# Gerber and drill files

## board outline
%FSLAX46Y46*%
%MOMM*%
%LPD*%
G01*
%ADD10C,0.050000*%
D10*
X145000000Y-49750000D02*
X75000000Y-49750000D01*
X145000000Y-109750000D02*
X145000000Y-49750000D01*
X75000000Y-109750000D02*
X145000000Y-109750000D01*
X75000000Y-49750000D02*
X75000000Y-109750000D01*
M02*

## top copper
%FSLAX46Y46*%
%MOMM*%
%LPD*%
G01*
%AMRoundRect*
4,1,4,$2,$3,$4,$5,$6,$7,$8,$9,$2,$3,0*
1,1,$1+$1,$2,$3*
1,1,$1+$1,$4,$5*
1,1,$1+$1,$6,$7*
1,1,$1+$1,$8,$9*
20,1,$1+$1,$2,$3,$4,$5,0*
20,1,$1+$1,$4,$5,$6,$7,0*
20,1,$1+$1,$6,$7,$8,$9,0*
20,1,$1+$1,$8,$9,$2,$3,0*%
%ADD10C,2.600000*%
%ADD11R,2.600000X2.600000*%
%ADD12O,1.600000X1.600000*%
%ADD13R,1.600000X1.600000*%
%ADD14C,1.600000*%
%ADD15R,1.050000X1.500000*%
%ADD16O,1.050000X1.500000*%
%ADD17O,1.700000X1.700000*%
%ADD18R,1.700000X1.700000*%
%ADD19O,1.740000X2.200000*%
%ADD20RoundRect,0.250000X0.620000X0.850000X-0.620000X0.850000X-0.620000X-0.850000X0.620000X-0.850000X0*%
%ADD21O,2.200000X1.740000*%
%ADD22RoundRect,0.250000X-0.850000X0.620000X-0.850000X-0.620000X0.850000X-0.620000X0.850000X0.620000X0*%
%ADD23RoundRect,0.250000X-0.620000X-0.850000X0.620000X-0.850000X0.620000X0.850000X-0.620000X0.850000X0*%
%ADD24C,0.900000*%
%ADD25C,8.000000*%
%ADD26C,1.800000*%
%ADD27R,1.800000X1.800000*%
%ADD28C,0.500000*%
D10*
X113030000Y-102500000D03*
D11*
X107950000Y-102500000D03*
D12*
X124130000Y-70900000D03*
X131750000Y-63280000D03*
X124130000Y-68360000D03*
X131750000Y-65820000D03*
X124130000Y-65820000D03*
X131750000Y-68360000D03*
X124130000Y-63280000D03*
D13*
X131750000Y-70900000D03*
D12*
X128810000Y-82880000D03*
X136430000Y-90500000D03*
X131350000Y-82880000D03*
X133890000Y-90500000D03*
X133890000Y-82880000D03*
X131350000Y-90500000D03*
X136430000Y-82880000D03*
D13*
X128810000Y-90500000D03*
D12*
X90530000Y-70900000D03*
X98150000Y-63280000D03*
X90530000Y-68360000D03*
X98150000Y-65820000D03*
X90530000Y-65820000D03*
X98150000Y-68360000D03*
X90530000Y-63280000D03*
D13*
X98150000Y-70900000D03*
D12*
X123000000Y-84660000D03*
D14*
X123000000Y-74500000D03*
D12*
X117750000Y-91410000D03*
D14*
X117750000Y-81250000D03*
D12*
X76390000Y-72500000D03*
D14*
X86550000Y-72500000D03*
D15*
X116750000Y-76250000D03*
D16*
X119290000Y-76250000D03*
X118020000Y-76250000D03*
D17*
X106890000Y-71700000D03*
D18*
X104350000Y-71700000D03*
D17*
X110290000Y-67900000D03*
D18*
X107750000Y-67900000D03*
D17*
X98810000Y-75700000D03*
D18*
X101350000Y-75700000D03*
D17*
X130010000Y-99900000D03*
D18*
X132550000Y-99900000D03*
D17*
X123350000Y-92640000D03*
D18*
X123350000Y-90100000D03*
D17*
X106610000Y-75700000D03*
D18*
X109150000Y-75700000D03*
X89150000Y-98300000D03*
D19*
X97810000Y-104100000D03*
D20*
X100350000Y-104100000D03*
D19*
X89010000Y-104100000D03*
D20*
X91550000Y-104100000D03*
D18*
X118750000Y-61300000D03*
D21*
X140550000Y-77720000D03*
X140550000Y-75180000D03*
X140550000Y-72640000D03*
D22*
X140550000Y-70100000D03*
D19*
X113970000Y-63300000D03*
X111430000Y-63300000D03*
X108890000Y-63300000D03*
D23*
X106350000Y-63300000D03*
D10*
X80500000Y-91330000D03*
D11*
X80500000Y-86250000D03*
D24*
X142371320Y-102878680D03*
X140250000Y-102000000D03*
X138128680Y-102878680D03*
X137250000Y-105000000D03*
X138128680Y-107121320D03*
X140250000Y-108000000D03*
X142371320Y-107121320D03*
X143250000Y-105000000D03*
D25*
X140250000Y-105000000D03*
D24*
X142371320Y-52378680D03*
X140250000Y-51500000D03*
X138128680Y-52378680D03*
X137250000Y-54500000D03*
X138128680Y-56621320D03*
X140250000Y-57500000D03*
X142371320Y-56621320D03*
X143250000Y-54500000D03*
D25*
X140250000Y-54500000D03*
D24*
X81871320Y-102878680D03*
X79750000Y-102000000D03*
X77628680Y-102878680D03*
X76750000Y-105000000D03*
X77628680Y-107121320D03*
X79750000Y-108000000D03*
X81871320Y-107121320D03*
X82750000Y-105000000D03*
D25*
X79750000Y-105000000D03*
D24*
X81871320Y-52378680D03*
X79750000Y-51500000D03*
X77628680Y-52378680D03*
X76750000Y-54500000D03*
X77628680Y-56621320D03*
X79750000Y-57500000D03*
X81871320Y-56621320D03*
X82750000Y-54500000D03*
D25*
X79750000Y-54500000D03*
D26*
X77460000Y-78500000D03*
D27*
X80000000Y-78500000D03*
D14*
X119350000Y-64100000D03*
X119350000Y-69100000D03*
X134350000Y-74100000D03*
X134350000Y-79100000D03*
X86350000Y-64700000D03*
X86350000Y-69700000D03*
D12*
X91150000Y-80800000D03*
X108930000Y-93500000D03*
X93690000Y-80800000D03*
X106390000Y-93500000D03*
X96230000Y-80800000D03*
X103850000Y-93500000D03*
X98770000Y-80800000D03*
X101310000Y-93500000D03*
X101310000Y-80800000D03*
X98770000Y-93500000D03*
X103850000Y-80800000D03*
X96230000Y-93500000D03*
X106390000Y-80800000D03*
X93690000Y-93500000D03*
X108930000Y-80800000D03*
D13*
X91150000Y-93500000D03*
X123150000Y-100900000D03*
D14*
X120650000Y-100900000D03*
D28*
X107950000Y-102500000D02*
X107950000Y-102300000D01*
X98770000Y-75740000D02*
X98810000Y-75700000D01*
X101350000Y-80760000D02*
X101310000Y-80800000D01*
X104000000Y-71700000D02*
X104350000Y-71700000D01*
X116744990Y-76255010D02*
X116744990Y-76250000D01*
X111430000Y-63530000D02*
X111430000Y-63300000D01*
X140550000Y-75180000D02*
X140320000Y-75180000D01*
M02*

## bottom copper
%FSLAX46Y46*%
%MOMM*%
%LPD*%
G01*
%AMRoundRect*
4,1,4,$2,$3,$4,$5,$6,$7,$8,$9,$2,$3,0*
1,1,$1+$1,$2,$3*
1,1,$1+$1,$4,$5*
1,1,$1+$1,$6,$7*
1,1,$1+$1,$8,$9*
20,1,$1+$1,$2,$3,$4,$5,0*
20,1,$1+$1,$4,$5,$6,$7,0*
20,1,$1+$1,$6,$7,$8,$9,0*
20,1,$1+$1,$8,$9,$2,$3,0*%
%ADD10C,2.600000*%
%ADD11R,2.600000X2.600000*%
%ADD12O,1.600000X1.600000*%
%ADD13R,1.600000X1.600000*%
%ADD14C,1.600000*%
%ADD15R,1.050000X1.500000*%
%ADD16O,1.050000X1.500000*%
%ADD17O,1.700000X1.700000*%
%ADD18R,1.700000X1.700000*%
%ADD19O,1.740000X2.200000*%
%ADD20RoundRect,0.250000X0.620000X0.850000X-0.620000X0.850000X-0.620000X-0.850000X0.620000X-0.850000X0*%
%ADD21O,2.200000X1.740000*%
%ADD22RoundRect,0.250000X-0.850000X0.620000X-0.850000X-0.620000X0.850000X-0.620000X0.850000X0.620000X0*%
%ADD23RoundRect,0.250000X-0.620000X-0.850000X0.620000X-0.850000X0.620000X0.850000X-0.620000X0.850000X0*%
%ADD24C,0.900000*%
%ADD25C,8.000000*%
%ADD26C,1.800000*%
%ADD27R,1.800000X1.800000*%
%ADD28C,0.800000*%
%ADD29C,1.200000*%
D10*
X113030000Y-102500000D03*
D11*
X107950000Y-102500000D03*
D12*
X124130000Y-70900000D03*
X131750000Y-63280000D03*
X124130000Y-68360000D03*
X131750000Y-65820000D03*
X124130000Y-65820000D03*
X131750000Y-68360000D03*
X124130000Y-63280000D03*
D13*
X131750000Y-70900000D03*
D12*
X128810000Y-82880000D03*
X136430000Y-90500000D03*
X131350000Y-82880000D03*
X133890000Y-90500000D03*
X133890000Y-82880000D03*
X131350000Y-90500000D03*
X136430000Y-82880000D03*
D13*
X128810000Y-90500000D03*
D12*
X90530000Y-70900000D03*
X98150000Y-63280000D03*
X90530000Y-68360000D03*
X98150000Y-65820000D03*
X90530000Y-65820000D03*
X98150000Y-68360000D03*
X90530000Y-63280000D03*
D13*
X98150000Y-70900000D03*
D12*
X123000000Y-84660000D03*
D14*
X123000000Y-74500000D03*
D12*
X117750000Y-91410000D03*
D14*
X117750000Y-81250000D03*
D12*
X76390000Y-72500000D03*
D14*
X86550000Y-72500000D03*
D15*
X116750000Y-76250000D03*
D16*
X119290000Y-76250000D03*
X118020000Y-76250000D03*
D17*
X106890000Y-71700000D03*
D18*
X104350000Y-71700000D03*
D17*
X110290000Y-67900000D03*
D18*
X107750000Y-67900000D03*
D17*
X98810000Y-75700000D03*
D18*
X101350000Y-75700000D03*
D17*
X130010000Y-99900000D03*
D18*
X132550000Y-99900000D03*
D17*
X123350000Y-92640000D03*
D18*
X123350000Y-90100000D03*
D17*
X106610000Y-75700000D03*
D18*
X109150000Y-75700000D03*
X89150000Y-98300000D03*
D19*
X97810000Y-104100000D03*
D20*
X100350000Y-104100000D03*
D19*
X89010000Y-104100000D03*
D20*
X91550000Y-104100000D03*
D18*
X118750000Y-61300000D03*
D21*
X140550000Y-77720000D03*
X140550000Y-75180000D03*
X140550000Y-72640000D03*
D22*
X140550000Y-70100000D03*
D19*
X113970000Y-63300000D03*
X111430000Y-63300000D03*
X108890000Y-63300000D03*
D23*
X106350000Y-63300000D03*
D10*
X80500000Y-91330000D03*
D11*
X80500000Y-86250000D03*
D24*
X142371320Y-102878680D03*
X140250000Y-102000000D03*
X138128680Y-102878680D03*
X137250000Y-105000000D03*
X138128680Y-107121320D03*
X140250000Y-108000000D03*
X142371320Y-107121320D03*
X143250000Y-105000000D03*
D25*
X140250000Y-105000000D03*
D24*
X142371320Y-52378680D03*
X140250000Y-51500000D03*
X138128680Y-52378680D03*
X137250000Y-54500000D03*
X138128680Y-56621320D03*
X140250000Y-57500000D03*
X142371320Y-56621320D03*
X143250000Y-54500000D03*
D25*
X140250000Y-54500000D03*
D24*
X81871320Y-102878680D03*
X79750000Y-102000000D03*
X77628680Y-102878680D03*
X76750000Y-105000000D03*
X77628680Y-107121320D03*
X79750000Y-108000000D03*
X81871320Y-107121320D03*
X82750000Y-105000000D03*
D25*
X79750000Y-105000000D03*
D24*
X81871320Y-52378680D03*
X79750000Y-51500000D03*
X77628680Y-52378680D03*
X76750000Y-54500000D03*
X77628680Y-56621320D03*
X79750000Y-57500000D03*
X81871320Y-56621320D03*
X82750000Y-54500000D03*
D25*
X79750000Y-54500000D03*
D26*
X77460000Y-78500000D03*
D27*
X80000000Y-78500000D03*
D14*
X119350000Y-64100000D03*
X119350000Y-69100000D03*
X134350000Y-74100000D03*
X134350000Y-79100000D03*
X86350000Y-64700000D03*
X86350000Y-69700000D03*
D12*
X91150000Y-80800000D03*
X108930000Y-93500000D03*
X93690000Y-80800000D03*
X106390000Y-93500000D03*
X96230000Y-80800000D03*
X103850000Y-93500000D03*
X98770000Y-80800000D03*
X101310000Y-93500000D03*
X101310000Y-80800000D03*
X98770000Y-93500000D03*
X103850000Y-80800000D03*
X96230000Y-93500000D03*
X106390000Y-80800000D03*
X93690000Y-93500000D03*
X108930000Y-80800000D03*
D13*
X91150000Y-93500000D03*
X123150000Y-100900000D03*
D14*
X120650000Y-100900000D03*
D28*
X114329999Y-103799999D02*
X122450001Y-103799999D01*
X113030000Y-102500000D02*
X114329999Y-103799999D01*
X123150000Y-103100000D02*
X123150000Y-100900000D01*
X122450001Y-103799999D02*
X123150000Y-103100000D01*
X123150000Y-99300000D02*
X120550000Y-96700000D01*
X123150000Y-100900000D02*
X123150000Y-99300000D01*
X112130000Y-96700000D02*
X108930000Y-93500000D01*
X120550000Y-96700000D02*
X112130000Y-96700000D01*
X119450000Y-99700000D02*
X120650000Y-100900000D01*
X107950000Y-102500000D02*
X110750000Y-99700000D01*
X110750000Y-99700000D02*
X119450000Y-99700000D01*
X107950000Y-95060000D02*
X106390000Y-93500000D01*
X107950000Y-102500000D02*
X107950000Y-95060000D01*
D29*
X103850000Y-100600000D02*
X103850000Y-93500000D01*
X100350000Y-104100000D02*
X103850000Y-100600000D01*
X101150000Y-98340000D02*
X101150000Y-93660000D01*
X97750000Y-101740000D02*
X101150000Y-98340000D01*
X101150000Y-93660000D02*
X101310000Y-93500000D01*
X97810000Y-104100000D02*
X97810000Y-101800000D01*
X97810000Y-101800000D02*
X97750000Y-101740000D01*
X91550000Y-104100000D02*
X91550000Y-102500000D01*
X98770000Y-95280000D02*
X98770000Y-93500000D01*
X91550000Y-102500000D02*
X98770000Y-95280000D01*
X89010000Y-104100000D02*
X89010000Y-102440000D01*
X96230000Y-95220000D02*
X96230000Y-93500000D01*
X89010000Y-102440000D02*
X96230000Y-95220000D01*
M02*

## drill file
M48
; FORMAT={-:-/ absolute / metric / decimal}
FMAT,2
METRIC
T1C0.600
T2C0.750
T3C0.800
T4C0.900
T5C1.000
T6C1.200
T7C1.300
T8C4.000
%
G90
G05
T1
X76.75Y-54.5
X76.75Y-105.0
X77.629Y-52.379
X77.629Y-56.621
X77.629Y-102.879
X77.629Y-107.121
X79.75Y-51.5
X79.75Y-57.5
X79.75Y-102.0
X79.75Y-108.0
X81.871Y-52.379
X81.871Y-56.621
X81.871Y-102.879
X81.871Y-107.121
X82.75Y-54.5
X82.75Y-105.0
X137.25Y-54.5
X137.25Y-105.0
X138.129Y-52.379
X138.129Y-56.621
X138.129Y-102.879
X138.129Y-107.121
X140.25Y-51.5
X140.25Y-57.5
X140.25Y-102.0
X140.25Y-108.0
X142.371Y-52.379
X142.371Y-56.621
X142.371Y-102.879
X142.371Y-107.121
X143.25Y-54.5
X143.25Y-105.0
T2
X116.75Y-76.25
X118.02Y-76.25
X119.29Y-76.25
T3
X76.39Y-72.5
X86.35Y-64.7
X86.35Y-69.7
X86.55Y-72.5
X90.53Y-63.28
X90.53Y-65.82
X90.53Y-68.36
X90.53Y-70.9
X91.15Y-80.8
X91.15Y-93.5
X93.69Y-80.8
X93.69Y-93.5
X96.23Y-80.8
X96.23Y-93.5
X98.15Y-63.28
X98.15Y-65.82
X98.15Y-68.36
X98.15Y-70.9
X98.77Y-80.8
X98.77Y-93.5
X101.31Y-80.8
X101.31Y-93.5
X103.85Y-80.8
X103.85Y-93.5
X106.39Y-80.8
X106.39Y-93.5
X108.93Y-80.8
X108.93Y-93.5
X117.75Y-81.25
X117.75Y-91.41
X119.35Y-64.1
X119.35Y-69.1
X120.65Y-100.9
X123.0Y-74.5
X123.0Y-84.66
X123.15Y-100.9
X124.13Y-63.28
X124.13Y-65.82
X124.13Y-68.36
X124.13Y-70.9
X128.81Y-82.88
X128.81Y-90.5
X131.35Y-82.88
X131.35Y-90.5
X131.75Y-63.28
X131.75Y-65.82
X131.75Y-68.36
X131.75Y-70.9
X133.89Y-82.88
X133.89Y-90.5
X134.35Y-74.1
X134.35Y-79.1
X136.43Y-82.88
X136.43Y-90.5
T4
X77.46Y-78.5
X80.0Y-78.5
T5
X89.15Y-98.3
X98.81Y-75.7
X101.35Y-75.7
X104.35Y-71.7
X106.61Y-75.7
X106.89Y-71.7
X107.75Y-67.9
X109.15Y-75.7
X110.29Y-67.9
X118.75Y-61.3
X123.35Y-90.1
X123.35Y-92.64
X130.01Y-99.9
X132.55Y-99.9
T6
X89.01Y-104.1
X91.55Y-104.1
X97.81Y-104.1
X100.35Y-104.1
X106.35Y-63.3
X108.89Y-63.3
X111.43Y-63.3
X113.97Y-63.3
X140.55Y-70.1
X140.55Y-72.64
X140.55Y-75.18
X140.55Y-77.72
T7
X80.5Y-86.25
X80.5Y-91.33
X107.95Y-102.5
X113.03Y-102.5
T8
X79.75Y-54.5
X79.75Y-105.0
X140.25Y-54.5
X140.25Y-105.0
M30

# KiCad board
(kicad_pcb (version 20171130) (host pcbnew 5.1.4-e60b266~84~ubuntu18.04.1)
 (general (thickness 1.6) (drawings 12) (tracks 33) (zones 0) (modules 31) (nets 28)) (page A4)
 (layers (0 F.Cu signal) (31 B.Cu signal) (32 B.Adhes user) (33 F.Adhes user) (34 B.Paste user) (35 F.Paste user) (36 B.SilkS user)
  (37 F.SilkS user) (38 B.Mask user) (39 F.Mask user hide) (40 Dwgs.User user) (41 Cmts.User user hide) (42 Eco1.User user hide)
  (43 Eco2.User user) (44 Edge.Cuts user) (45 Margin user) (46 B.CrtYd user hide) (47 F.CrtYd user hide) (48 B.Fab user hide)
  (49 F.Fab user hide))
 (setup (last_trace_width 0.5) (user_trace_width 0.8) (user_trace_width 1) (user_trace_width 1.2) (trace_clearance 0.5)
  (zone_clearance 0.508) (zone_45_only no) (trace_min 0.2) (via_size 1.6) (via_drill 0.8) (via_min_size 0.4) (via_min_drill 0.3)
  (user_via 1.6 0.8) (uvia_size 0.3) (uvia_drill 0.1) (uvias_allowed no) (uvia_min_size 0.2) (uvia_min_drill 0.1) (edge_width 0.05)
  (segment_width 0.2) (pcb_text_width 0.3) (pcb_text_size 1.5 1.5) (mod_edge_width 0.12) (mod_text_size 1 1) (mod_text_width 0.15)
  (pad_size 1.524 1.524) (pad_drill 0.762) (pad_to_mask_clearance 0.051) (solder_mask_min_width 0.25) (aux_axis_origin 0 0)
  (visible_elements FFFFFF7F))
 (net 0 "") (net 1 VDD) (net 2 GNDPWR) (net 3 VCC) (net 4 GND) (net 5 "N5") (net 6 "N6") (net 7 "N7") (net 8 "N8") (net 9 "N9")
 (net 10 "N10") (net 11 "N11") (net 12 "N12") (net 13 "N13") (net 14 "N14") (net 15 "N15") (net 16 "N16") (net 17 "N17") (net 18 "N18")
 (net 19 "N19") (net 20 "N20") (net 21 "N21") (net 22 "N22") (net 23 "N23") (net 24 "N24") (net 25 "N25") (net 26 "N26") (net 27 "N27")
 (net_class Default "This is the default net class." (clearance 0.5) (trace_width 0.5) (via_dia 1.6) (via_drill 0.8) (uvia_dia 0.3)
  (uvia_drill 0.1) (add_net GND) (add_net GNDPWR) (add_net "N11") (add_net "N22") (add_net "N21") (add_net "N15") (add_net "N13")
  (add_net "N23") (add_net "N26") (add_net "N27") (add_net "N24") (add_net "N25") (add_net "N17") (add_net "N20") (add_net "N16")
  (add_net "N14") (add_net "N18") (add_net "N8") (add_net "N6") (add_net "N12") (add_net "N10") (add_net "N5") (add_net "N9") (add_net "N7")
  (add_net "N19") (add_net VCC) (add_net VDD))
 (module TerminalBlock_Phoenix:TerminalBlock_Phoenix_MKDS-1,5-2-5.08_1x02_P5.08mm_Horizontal (layer F.Cu) (at 107.95 102.5)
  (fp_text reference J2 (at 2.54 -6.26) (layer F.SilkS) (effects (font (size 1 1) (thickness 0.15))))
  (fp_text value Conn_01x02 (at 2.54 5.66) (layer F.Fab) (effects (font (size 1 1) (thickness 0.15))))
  (pad 2 thru_hole circle (at 5.08 0) (size 2.6 2.6) (drill 1.3) (layers *.Cu *.Mask) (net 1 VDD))
  (pad 1 thru_hole rect (at 0 0) (size 2.6 2.6) (drill 1.3) (layers *.Cu *.Mask) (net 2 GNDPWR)))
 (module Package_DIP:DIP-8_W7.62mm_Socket (layer F.Cu) (at 131.75 70.9 180)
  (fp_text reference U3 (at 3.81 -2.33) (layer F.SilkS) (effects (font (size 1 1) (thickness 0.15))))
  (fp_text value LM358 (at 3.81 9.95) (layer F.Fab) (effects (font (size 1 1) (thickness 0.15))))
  (pad 8 thru_hole oval (at 7.62 0 180) (size 1.6 1.6) (drill 0.8) (layers *.Cu *.Mask) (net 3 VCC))
  (pad 4 thru_hole oval (at 0 7.62 180) (size 1.6 1.6) (drill 0.8) (layers *.Cu *.Mask) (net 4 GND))
  (pad 7 thru_hole oval (at 7.62 2.54 180) (size 1.6 1.6) (drill 0.8) (layers *.Cu *.Mask) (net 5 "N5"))
  (pad 3 thru_hole oval (at 0 5.08 180) (size 1.6 1.6) (drill 0.8) (layers *.Cu *.Mask) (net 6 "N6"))
  (pad 6 thru_hole oval (at 7.62 5.08 180) (size 1.6 1.6) (drill 0.8) (layers *.Cu *.Mask) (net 5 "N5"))
  (pad 2 thru_hole oval (at 0 2.54 180) (size 1.6 1.6) (drill 0.8) (layers *.Cu *.Mask) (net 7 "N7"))
  (pad 5 thru_hole oval (at 7.62 7.62 180) (size 1.6 1.6) (drill 0.8) (layers *.Cu *.Mask) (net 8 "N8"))
  (pad 1 thru_hole rect (at 0 0 180) (size 1.6 1.6) (drill 0.8) (layers *.Cu *.Mask) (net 7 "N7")))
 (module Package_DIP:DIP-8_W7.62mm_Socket (layer F.Cu) (at 128.81 90.5 90)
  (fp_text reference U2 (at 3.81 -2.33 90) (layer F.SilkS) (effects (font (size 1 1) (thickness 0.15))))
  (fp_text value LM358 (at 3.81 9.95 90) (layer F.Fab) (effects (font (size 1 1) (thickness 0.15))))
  (pad 8 thru_hole oval (at 7.62 0 90) (size 1.6 1.6) (drill 0.8) (layers *.Cu *.Mask) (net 3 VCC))
  (pad 4 thru_hole oval (at 0 7.62 90) (size 1.6 1.6) (drill 0.8) (layers *.Cu *.Mask) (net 4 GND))
  (pad 7 thru_hole oval (at 7.62 2.54 90) (size 1.6 1.6) (drill 0.8) (layers *.Cu *.Mask) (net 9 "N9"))
  (pad 3 thru_hole oval (at 0 5.08 90) (size 1.6 1.6) (drill 0.8) (layers *.Cu *.Mask) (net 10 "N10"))
  (pad 6 thru_hole oval (at 7.62 5.08 90) (size 1.6 1.6) (drill 0.8) (layers *.Cu *.Mask) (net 9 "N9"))
  (pad 2 thru_hole oval (at 0 2.54 90) (size 1.6 1.6) (drill 0.8) (layers *.Cu *.Mask) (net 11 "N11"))
  (pad 5 thru_hole oval (at 7.62 7.62 90) (size 1.6 1.6) (drill 0.8) (layers *.Cu *.Mask) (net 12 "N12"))
  (pad 1 thru_hole rect (at 0 0 90) (size 1.6 1.6) (drill 0.8) (layers *.Cu *.Mask) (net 11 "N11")))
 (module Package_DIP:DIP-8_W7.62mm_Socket (layer F.Cu) (at 98.15 70.9 180)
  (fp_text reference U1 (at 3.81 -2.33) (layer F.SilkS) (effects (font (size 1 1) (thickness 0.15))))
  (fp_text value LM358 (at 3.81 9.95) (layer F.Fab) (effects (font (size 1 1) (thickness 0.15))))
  (pad 8 thru_hole oval (at 7.62 0 180) (size 1.6 1.6) (drill 0.8) (layers *.Cu *.Mask) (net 3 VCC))
  (pad 4 thru_hole oval (at 0 7.62 180) (size 1.6 1.6) (drill 0.8) (layers *.Cu *.Mask) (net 4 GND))
  (pad 7 thru_hole oval (at 7.62 2.54 180) (size 1.6 1.6) (drill 0.8) (layers *.Cu *.Mask) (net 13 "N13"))
  (pad 3 thru_hole oval (at 0 5.08 180) (size 1.6 1.6) (drill 0.8) (layers *.Cu *.Mask) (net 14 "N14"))
  (pad 6 thru_hole oval (at 7.62 5.08 180) (size 1.6 1.6) (drill 0.8) (layers *.Cu *.Mask) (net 13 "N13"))
  (pad 2 thru_hole oval (at 0 2.54 180) (size 1.6 1.6) (drill 0.8) (layers *.Cu *.Mask) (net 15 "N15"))
  (pad 5 thru_hole oval (at 7.62 7.62 180) (size 1.6 1.6) (drill 0.8) (layers *.Cu *.Mask) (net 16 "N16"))
  (pad 1 thru_hole rect (at 0 0 180) (size 1.6 1.6) (drill 0.8) (layers *.Cu *.Mask) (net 15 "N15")))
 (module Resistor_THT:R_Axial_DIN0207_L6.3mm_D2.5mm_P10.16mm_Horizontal (layer F.Cu) (at 123 74.5 270)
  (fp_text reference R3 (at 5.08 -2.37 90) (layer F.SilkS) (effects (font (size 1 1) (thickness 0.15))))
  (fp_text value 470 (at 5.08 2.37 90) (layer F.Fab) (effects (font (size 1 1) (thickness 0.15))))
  (pad 2 thru_hole oval (at 10.16 0 270) (size 1.6 1.6) (drill 0.8) (layers *.Cu *.Mask) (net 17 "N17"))
  (pad 1 thru_hole circle (at 0 0 270) (size 1.6 1.6) (drill 0.8) (layers *.Cu *.Mask) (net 3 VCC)))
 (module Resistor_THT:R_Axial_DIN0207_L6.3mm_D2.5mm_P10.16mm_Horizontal (layer F.Cu) (at 117.75 81.25 270)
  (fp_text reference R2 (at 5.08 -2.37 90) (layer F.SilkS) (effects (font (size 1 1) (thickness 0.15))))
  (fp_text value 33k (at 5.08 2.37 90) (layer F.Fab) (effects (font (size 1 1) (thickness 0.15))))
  (pad 2 thru_hole oval (at 10.16 0 270) (size 1.6 1.6) (drill 0.8) (layers *.Cu *.Mask) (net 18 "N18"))
  (pad 1 thru_hole circle (at 0 0 270) (size 1.6 1.6) (drill 0.8) (layers *.Cu *.Mask) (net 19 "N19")))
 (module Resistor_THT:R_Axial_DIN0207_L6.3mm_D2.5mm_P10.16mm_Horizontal (layer F.Cu) (at 86.55 72.5 180)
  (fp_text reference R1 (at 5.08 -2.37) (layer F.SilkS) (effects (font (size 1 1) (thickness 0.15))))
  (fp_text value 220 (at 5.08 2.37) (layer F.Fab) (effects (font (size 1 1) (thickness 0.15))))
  (pad 2 thru_hole oval (at 10.16 0 180) (size 1.6 1.6) (drill 0.8) (layers *.Cu *.Mask) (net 4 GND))
  (pad 1 thru_hole circle (at 0 0 180) (size 1.6 1.6) (drill 0.8) (layers *.Cu *.Mask) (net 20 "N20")))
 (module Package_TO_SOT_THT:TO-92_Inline (layer F.Cu) (at 116.75 76.25)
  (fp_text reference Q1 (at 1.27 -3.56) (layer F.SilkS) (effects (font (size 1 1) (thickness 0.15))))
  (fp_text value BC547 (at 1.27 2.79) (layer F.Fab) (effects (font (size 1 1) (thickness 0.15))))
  (pad 1 thru_hole rect (at 0 0) (size 1.05 1.5) (drill 0.75) (layers *.Cu *.Mask) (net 17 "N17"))
  (pad 3 thru_hole oval (at 2.54 0) (size 1.05 1.5) (drill 0.75) (layers *.Cu *.Mask) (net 4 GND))
  (pad 2 thru_hole oval (at 1.27 0) (size 1.05 1.5) (drill 0.75) (layers *.Cu *.Mask) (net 19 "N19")))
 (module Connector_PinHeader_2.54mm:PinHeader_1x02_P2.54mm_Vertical (layer F.Cu) (at 104.35 71.7 90)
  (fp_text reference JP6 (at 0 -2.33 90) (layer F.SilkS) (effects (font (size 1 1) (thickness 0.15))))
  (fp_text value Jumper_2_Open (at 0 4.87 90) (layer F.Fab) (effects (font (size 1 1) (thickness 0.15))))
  (pad 2 thru_hole oval (at 0 2.54 90) (size 1.7 1.7) (drill 1) (layers *.Cu *.Mask) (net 7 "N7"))
  (pad 1 thru_hole rect (at 0 0 90) (size 1.7 1.7) (drill 1) (layers *.Cu *.Mask) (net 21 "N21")))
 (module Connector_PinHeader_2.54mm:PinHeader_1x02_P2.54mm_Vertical (layer F.Cu) (at 107.75 67.9 90)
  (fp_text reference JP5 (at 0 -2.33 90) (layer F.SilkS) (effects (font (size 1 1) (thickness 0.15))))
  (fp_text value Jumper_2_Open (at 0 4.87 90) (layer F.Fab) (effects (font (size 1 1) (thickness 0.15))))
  (pad 2 thru_hole oval (at 0 2.54 90) (size 1.7 1.7) (drill 1) (layers *.Cu *.Mask) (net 4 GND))
  (pad 1 thru_hole rect (at 0 0 90) (size 1.7 1.7) (drill 1) (layers *.Cu *.Mask) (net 21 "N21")))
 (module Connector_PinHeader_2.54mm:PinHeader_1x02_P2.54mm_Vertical (layer F.Cu) (at 101.35 75.7 270)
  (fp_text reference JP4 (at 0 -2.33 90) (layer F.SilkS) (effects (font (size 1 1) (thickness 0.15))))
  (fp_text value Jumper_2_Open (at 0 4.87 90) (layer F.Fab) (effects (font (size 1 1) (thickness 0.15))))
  (pad 2 thru_hole oval (at 0 2.54 270) (size 1.7 1.7) (drill 1) (layers *.Cu *.Mask) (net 3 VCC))
  (pad 1 thru_hole rect (at 0 0 270) (size 1.7 1.7) (drill 1) (layers *.Cu *.Mask) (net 21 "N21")))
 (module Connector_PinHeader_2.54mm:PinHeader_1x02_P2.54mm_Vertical (layer F.Cu) (at 132.55 99.9 270)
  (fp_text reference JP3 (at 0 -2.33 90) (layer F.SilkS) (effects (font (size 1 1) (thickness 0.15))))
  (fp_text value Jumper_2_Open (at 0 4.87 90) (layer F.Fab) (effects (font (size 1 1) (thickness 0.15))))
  (pad 2 thru_hole oval (at 0 2.54 270) (size 1.7 1.7) (drill 1) (layers *.Cu *.Mask) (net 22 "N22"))
  (pad 1 thru_hole rect (at 0 0 270) (size 1.7 1.7) (drill 1) (layers *.Cu *.Mask) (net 4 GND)))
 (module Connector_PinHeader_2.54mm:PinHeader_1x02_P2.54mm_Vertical (layer F.Cu) (at 123.35 90.1)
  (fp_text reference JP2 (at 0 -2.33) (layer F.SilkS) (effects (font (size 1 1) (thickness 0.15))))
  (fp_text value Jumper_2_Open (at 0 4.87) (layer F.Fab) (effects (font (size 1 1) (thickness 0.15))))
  (pad 2 thru_hole oval (at 0 2.54) (size 1.7 1.7) (drill 1) (layers *.Cu *.Mask) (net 22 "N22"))
  (pad 1 thru_hole rect (at 0 0) (size 1.7 1.7) (drill 1) (layers *.Cu *.Mask) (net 9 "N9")))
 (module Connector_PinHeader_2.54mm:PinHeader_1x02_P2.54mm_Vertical (layer F.Cu) (at 109.15 75.7 270)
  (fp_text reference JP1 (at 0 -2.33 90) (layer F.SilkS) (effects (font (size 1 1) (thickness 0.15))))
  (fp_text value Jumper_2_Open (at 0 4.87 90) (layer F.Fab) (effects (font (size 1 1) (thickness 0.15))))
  (pad 2 thru_hole oval (at 0 2.54 270) (size 1.7 1.7) (drill 1) (layers *.Cu *.Mask) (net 22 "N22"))
  (pad 1 thru_hole rect (at 0 0 270) (size 1.7 1.7) (drill 1) (layers *.Cu *.Mask) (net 3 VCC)))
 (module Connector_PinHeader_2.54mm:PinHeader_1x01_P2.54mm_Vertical (layer F.Cu) (at 89.15 98.3 90)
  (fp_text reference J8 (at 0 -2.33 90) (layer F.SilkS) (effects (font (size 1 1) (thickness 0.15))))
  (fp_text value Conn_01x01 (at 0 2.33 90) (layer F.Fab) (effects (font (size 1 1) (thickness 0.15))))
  (pad 1 thru_hole rect (at 0 0 90) (size 1.7 1.7) (drill 1) (layers *.Cu *.Mask) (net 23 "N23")))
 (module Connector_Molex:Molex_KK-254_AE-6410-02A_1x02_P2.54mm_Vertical (layer F.Cu) (at 100.35 104.1 180)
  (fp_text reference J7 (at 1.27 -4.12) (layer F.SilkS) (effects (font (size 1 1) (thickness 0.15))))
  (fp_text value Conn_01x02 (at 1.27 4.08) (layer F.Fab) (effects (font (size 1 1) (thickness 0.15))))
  (pad 2 thru_hole oval (at 2.54 0 180) (size 1.74 2.2) (drill 1.2) (layers *.Cu *.Mask) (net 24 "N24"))
  (pad 1 thru_hole roundrect (at 0 0 180) (size 1.74 2.2) (drill 1.2) (layers *.Cu *.Mask) (roundrect_rratio 0.143678) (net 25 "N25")))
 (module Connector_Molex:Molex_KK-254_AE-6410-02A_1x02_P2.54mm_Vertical (layer F.Cu) (at 91.55 104.1 180)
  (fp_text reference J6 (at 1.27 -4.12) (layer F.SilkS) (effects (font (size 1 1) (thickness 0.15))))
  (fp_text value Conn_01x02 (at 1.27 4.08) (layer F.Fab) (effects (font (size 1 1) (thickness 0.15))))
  (pad 2 thru_hole oval (at 2.54 0 180) (size 1.74 2.2) (drill 1.2) (layers *.Cu *.Mask) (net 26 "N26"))
  (pad 1 thru_hole roundrect (at 0 0 180) (size 1.74 2.2) (drill 1.2) (layers *.Cu *.Mask) (roundrect_rratio 0.143678) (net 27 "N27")))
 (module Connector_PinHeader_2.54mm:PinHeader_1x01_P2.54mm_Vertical (layer F.Cu) (at 118.75 61.3 90)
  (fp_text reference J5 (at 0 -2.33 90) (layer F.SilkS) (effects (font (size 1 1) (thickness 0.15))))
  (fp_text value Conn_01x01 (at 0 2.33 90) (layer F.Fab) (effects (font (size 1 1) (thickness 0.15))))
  (pad 1 thru_hole rect (at 0 0 90) (size 1.7 1.7) (drill 1) (layers *.Cu *.Mask) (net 5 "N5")))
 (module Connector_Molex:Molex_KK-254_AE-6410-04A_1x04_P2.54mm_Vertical (layer F.Cu) (at 140.55 70.1 270)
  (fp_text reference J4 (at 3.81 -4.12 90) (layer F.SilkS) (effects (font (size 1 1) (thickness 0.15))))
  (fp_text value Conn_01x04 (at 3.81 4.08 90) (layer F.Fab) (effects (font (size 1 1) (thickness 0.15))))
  (pad 4 thru_hole oval (at 7.62 0 270) (size 1.74 2.2) (drill 1.2) (layers *.Cu *.Mask) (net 10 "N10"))
  (pad 3 thru_hole oval (at 5.08 0 270) (size 1.74 2.2) (drill 1.2) (layers *.Cu *.Mask) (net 12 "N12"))
  (pad 2 thru_hole oval (at 2.54 0 270) (size 1.74 2.2) (drill 1.2) (layers *.Cu *.Mask) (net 6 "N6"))
  (pad 1 thru_hole roundrect (at 0 0 270) (size 1.74 2.2) (drill 1.2) (layers *.Cu *.Mask) (roundrect_rratio 0.143678) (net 8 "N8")))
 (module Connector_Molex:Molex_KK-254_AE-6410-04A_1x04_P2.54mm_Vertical (layer F.Cu) (at 106.35 63.3)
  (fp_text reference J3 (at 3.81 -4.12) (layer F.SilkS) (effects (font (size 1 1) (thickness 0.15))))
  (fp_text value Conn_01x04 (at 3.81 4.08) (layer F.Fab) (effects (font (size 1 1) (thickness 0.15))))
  (pad 4 thru_hole oval (at 7.62 0) (size 1.74 2.2) (drill 1.2) (layers *.Cu *.Mask) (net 18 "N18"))
  (pad 3 thru_hole oval (at 5.08 0) (size 1.74 2.2) (drill 1.2) (layers *.Cu *.Mask) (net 14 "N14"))
  (pad 2 thru_hole oval (at 2.54 0) (size 1.74 2.2) (drill 1.2) (layers *.Cu *.Mask) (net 16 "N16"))
  (pad 1 thru_hole roundrect (at 0 0) (size 1.74 2.2) (drill 1.2) (layers *.Cu *.Mask) (roundrect_rratio 0.143678) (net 4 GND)))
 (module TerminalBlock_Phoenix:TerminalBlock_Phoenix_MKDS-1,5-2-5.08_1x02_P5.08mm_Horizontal (layer F.Cu) (at 80.5 86.25 270)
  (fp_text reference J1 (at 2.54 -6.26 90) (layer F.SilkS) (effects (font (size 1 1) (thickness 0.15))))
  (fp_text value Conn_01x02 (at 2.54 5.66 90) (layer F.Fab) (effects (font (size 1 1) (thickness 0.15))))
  (pad 2 thru_hole circle (at 5.08 0 270) (size 2.6 2.6) (drill 1.3) (layers *.Cu *.Mask) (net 3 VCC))
  (pad 1 thru_hole rect (at 0 0 270) (size 2.6 2.6) (drill 1.3) (layers *.Cu *.Mask) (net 4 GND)))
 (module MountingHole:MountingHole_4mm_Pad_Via (layer F.Cu) (at 140.25 105)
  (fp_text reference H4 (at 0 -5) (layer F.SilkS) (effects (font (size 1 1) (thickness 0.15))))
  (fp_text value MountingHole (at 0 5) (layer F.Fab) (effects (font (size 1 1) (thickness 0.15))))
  (pad 1 thru_hole circle (at 2.12132 -2.12132) (size 0.9 0.9) (drill 0.6) (layers *.Cu *.Mask))
  (pad 1 thru_hole circle (at 0 -3) (size 0.9 0.9) (drill 0.6) (layers *.Cu *.Mask))
  (pad 1 thru_hole circle (at -2.12132 -2.12132) (size 0.9 0.9) (drill 0.6) (layers *.Cu *.Mask))
  (pad 1 thru_hole circle (at -3 0) (size 0.9 0.9) (drill 0.6) (layers *.Cu *.Mask))
  (pad 1 thru_hole circle (at -2.12132 2.12132) (size 0.9 0.9) (drill 0.6) (layers *.Cu *.Mask))
  (pad 1 thru_hole circle (at 0 3) (size 0.9 0.9) (drill 0.6) (layers *.Cu *.Mask))
  (pad 1 thru_hole circle (at 2.12132 2.12132) (size 0.9 0.9) (drill 0.6) (layers *.Cu *.Mask))
  (pad 1 thru_hole circle (at 3 0) (size 0.9 0.9) (drill 0.6) (layers *.Cu *.Mask))
  (pad 1 thru_hole circle (at 0 0) (size 8 8) (drill 4) (layers *.Cu *.Mask)))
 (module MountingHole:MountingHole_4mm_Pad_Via (layer F.Cu) (at 140.25 54.5)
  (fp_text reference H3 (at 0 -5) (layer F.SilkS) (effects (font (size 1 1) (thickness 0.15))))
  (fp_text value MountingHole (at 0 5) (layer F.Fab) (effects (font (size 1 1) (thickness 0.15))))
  (pad 1 thru_hole circle (at 2.12132 -2.12132) (size 0.9 0.9) (drill 0.6) (layers *.Cu *.Mask))
  (pad 1 thru_hole circle (at 0 -3) (size 0.9 0.9) (drill 0.6) (layers *.Cu *.Mask))
  (pad 1 thru_hole circle (at -2.12132 -2.12132) (size 0.9 0.9) (drill 0.6) (layers *.Cu *.Mask))
  (pad 1 thru_hole circle (at -3 0) (size 0.9 0.9) (drill 0.6) (layers *.Cu *.Mask))
  (pad 1 thru_hole circle (at -2.12132 2.12132) (size 0.9 0.9) (drill 0.6) (layers *.Cu *.Mask))
  (pad 1 thru_hole circle (at 0 3) (size 0.9 0.9) (drill 0.6) (layers *.Cu *.Mask))
  (pad 1 thru_hole circle (at 2.12132 2.12132) (size 0.9 0.9) (drill 0.6) (layers *.Cu *.Mask))
  (pad 1 thru_hole circle (at 3 0) (size 0.9 0.9) (drill 0.6) (layers *.Cu *.Mask))
  (pad 1 thru_hole circle (at 0 0) (size 8 8) (drill 4) (layers *.Cu *.Mask)))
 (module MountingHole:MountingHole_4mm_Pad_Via (layer F.Cu) (at 79.75 105)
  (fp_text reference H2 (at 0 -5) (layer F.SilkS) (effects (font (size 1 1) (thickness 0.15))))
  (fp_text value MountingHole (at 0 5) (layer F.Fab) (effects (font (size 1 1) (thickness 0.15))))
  (pad 1 thru_hole circle (at 2.12132 -2.12132) (size 0.9 0.9) (drill 0.6) (layers *.Cu *.Mask))
  (pad 1 thru_hole circle (at 0 -3) (size 0.9 0.9) (drill 0.6) (layers *.Cu *.Mask))
  (pad 1 thru_hole circle (at -2.12132 -2.12132) (size 0.9 0.9) (drill 0.6) (layers *.Cu *.Mask))
  (pad 1 thru_hole circle (at -3 0) (size 0.9 0.9) (drill 0.6) (layers *.Cu *.Mask))
  (pad 1 thru_hole circle (at -2.12132 2.12132) (size 0.9 0.9) (drill 0.6) (layers *.Cu *.Mask))
  (pad 1 thru_hole circle (at 0 3) (size 0.9 0.9) (drill 0.6) (layers *.Cu *.Mask))
  (pad 1 thru_hole circle (at 2.12132 2.12132) (size 0.9 0.9) (drill 0.6) (layers *.Cu *.Mask))
  (pad 1 thru_hole circle (at 3 0) (size 0.9 0.9) (drill 0.6) (layers *.Cu *.Mask))
  (pad 1 thru_hole circle (at 0 0) (size 8 8) (drill 4) (layers *.Cu *.Mask)))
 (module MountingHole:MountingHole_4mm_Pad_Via (layer F.Cu) (at 79.75 54.5)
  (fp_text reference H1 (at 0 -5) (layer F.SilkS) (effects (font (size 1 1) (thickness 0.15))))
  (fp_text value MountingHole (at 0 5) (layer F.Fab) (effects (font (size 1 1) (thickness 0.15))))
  (pad 1 thru_hole circle (at 2.12132 -2.12132) (size 0.9 0.9) (drill 0.6) (layers *.Cu *.Mask))
  (pad 1 thru_hole circle (at 0 -3) (size 0.9 0.9) (drill 0.6) (layers *.Cu *.Mask))
  (pad 1 thru_hole circle (at -2.12132 -2.12132) (size 0.9 0.9) (drill 0.6) (layers *.Cu *.Mask))
  (pad 1 thru_hole circle (at -3 0) (size 0.9 0.9) (drill 0.6) (layers *.Cu *.Mask))
  (pad 1 thru_hole circle (at -2.12132 2.12132) (size 0.9 0.9) (drill 0.6) (layers *.Cu *.Mask))
  (pad 1 thru_hole circle (at 0 3) (size 0.9 0.9) (drill 0.6) (layers *.Cu *.Mask))
  (pad 1 thru_hole circle (at 2.12132 2.12132) (size 0.9 0.9) (drill 0.6) (layers *.Cu *.Mask))
  (pad 1 thru_hole circle (at 3 0) (size 0.9 0.9) (drill 0.6) (layers *.Cu *.Mask))
  (pad 1 thru_hole circle (at 0 0) (size 8 8) (drill 4) (layers *.Cu *.Mask)))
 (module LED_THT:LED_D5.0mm (layer F.Cu) (at 80 78.5 180)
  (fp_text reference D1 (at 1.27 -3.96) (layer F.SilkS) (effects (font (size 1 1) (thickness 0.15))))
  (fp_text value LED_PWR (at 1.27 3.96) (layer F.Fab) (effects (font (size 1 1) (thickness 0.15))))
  (pad 2 thru_hole circle (at 2.54 0 180) (size 1.8 1.8) (drill 0.9) (layers *.Cu *.Mask) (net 3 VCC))
  (pad 1 thru_hole rect (at 0 0 180) (size 1.8 1.8) (drill 0.9) (layers *.Cu *.Mask) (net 20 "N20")))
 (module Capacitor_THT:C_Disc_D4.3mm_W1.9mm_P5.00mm (layer F.Cu) (at 119.35 69.1 90)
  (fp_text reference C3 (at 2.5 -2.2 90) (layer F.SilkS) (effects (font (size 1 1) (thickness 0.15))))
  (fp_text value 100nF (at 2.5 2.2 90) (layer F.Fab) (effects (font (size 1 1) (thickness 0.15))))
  (pad 2 thru_hole circle (at 5 0 90) (size 1.6 1.6) (drill 0.8) (layers *.Cu *.Mask) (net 4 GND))
  (pad 1 thru_hole circle (at 0 0 90) (size 1.6 1.6) (drill 0.8) (layers *.Cu *.Mask) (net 3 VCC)))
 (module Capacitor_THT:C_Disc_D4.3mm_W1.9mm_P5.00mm (layer F.Cu) (at 134.35 79.1 90)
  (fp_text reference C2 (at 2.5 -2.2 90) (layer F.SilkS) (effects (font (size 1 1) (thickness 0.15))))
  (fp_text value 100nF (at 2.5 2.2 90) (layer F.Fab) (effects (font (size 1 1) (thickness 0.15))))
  (pad 2 thru_hole circle (at 5 0 90) (size 1.6 1.6) (drill 0.8) (layers *.Cu *.Mask) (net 4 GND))
  (pad 1 thru_hole circle (at 0 0 90) (size 1.6 1.6) (drill 0.8) (layers *.Cu *.Mask) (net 3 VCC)))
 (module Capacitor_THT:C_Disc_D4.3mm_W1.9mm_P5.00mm (layer F.Cu) (at 86.35 69.7 90)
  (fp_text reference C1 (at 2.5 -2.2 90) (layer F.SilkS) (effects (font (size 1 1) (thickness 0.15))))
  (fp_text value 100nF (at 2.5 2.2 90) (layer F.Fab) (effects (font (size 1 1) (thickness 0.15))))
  (pad 2 thru_hole circle (at 5 0 90) (size 1.6 1.6) (drill 0.8) (layers *.Cu *.Mask) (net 4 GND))
  (pad 1 thru_hole circle (at 0 0 90) (size 1.6 1.6) (drill 0.8) (layers *.Cu *.Mask) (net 3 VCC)))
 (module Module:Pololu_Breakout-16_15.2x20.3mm (layer F.Cu) (at 91.15 93.5 90)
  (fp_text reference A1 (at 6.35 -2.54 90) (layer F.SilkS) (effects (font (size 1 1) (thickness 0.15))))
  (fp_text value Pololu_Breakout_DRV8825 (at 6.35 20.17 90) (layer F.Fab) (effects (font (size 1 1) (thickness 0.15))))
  (pad 16 thru_hole oval (at 12.7 0 90) (size 1.6 1.6) (drill 0.8) (layers *.Cu *.Mask) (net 13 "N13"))
  (pad 8 thru_hole oval (at 0 17.78 90) (size 1.6 1.6) (drill 0.8) (layers *.Cu *.Mask) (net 1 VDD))
  (pad 15 thru_hole oval (at 12.7 2.54 90) (size 1.6 1.6) (drill 0.8) (layers *.Cu *.Mask) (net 15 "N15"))
  (pad 7 thru_hole oval (at 0 15.24 90) (size 1.6 1.6) (drill 0.8) (layers *.Cu *.Mask) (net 2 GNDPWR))
  (pad 14 thru_hole oval (at 12.7 5.08 90) (size 1.6 1.6) (drill 0.8) (layers *.Cu *.Mask) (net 3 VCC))
  (pad 6 thru_hole oval (at 0 12.7 90) (size 1.6 1.6) (drill 0.8) (layers *.Cu *.Mask) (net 25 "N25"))
  (pad 13 thru_hole oval (at 12.7 7.62 90) (size 1.6 1.6) (drill 0.8) (layers *.Cu *.Mask) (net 3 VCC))
  (pad 5 thru_hole oval (at 0 10.16 90) (size 1.6 1.6) (drill 0.8) (layers *.Cu *.Mask) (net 24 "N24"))
  (pad 12 thru_hole oval (at 12.7 10.16 90) (size 1.6 1.6) (drill 0.8) (layers *.Cu *.Mask) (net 21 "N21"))
  (pad 4 thru_hole oval (at 0 7.62 90) (size 1.6 1.6) (drill 0.8) (layers *.Cu *.Mask) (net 27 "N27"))
  (pad 11 thru_hole oval (at 12.7 12.7 90) (size 1.6 1.6) (drill 0.8) (layers *.Cu *.Mask) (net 22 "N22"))
  (pad 3 thru_hole oval (at 0 5.08 90) (size 1.6 1.6) (drill 0.8) (layers *.Cu *.Mask) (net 26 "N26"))
  (pad 10 thru_hole oval (at 12.7 15.24 90) (size 1.6 1.6) (drill 0.8) (layers *.Cu *.Mask) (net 11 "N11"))
  (pad 2 thru_hole oval (at 0 2.54 90) (size 1.6 1.6) (drill 0.8) (layers *.Cu *.Mask) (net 23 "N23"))
  (pad 9 thru_hole oval (at 12.7 17.78 90) (size 1.6 1.6) (drill 0.8) (layers *.Cu *.Mask) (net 17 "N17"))
  (pad 1 thru_hole rect (at 0 0 90) (size 1.6 1.6) (drill 0.8) (layers *.Cu *.Mask) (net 4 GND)))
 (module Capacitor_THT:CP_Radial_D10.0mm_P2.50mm (layer F.Cu) (at 123.15 100.9 180)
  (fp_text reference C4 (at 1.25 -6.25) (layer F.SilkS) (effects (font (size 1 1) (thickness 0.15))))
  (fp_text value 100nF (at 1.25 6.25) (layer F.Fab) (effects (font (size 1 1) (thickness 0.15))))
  (pad 1 thru_hole rect (at 0 0 180) (size 1.6 1.6) (drill 0.8) (layers *.Cu *.Mask) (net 1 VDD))
  (pad 2 thru_hole circle (at 2.5 0 180) (size 1.6 1.6) (drill 0.8) (layers *.Cu *.Mask) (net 2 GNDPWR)))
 (gr_line (start 145 49.75) (end 75 49.75) (layer Edge.Cuts) (width 0.05))
 (gr_line (start 145 109.75) (end 145 49.75) (layer Edge.Cuts) (width 0.05))
 (gr_line (start 75 109.75) (end 145 109.75) (layer Edge.Cuts) (width 0.05))
 (gr_line (start 75 49.75) (end 75 109.75) (layer Edge.Cuts) (width 0.05))
 (segment (start 114.329999 103.799999) (end 122.450001 103.799999) (width 0.8) (layer B.Cu) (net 1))
 (segment (start 113.03 102.5) (end 114.329999 103.799999) (width 0.8) (layer B.Cu) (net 1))
 (segment (start 123.15 103.1) (end 123.15 100.9) (width 0.8) (layer B.Cu) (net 1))
 (segment (start 122.450001 103.799999) (end 123.15 103.1) (width 0.8) (layer B.Cu) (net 1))
 (segment (start 123.15 99.3) (end 120.55 96.7) (width 0.8) (layer B.Cu) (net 1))
 (segment (start 123.15 100.9) (end 123.15 99.3) (width 0.8) (layer B.Cu) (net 1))
 (segment (start 112.13 96.7) (end 108.93 93.5) (width 0.8) (layer B.Cu) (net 1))
 (segment (start 120.55 96.7) (end 112.13 96.7) (width 0.8) (layer B.Cu) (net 1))
 (segment (start 107.95 102.5) (end 107.95 102.3) (width 0.5) (layer F.Cu) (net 2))
 (segment (start 119.45 99.7) (end 120.65 100.9) (width 0.8) (layer B.Cu) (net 2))
 (segment (start 107.95 102.5) (end 110.75 99.7) (width 0.8) (layer B.Cu) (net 2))
 (segment (start 110.75 99.7) (end 119.45 99.7) (width 0.8) (layer B.Cu) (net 2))
 (segment (start 107.95 95.06) (end 106.39 93.5) (width 0.8) (layer B.Cu) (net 2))
 (segment (start 107.95 102.5) (end 107.95 95.06) (width 0.8) (layer B.Cu) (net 2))
 (segment (start 98.77 75.74) (end 98.81 75.7) (width 0.5) (layer F.Cu) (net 3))
 (segment (start 103.85 100.6) (end 103.85 93.5) (width 1.2) (layer B.Cu) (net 25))
 (segment (start 100.35 104.1) (end 103.85 100.6) (width 1.2) (layer B.Cu) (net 25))
 (segment (start 101.15 98.34) (end 101.15 93.66) (width 1.2) (layer B.Cu) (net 24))
 (segment (start 97.75 101.74) (end 101.15 98.34) (width 1.2) (layer B.Cu) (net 24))
 (segment (start 101.15 93.66) (end 101.31 93.5) (width 1.2) (layer B.Cu) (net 24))
 (segment (start 97.81 104.1) (end 97.81 101.8) (width 1.2) (layer B.Cu) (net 24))
 (segment (start 97.81 101.8) (end 97.75 101.74) (width 1.2) (layer B.Cu) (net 24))
 (segment (start 101.35 80.76) (end 101.31 80.8) (width 0.5) (layer F.Cu) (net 21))
 (segment (start 104 71.7) (end 104.35 71.7) (width 0.5) (layer F.Cu) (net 21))
 (segment (start 91.55 104.1) (end 91.55 102.5) (width 1.2) (layer B.Cu) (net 27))
 (segment (start 98.77 95.28) (end 98.77 93.5) (width 1.2) (layer B.Cu) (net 27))
 (segment (start 91.55 102.5) (end 98.77 95.28) (width 1.2) (layer B.Cu) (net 27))
 (segment (start 89.01 104.1) (end 89.01 102.44) (width 1.2) (layer B.Cu) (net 26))
 (segment (start 96.23 95.22) (end 96.23 93.5) (width 1.2) (layer B.Cu) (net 26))
 (segment (start 89.01 102.44) (end 96.23 95.22) (width 1.2) (layer B.Cu) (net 26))
 (segment (start 116.74499 76.25501) (end 116.74499 76.25) (width 0.5) (layer F.Cu) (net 17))
 (segment (start 111.43 63.53) (end 111.43 63.3) (width 0.5) (layer F.Cu) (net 14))
 (segment (start 140.55 75.18) (end 140.32 75.18) (width 0.5) (layer F.Cu) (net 12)))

